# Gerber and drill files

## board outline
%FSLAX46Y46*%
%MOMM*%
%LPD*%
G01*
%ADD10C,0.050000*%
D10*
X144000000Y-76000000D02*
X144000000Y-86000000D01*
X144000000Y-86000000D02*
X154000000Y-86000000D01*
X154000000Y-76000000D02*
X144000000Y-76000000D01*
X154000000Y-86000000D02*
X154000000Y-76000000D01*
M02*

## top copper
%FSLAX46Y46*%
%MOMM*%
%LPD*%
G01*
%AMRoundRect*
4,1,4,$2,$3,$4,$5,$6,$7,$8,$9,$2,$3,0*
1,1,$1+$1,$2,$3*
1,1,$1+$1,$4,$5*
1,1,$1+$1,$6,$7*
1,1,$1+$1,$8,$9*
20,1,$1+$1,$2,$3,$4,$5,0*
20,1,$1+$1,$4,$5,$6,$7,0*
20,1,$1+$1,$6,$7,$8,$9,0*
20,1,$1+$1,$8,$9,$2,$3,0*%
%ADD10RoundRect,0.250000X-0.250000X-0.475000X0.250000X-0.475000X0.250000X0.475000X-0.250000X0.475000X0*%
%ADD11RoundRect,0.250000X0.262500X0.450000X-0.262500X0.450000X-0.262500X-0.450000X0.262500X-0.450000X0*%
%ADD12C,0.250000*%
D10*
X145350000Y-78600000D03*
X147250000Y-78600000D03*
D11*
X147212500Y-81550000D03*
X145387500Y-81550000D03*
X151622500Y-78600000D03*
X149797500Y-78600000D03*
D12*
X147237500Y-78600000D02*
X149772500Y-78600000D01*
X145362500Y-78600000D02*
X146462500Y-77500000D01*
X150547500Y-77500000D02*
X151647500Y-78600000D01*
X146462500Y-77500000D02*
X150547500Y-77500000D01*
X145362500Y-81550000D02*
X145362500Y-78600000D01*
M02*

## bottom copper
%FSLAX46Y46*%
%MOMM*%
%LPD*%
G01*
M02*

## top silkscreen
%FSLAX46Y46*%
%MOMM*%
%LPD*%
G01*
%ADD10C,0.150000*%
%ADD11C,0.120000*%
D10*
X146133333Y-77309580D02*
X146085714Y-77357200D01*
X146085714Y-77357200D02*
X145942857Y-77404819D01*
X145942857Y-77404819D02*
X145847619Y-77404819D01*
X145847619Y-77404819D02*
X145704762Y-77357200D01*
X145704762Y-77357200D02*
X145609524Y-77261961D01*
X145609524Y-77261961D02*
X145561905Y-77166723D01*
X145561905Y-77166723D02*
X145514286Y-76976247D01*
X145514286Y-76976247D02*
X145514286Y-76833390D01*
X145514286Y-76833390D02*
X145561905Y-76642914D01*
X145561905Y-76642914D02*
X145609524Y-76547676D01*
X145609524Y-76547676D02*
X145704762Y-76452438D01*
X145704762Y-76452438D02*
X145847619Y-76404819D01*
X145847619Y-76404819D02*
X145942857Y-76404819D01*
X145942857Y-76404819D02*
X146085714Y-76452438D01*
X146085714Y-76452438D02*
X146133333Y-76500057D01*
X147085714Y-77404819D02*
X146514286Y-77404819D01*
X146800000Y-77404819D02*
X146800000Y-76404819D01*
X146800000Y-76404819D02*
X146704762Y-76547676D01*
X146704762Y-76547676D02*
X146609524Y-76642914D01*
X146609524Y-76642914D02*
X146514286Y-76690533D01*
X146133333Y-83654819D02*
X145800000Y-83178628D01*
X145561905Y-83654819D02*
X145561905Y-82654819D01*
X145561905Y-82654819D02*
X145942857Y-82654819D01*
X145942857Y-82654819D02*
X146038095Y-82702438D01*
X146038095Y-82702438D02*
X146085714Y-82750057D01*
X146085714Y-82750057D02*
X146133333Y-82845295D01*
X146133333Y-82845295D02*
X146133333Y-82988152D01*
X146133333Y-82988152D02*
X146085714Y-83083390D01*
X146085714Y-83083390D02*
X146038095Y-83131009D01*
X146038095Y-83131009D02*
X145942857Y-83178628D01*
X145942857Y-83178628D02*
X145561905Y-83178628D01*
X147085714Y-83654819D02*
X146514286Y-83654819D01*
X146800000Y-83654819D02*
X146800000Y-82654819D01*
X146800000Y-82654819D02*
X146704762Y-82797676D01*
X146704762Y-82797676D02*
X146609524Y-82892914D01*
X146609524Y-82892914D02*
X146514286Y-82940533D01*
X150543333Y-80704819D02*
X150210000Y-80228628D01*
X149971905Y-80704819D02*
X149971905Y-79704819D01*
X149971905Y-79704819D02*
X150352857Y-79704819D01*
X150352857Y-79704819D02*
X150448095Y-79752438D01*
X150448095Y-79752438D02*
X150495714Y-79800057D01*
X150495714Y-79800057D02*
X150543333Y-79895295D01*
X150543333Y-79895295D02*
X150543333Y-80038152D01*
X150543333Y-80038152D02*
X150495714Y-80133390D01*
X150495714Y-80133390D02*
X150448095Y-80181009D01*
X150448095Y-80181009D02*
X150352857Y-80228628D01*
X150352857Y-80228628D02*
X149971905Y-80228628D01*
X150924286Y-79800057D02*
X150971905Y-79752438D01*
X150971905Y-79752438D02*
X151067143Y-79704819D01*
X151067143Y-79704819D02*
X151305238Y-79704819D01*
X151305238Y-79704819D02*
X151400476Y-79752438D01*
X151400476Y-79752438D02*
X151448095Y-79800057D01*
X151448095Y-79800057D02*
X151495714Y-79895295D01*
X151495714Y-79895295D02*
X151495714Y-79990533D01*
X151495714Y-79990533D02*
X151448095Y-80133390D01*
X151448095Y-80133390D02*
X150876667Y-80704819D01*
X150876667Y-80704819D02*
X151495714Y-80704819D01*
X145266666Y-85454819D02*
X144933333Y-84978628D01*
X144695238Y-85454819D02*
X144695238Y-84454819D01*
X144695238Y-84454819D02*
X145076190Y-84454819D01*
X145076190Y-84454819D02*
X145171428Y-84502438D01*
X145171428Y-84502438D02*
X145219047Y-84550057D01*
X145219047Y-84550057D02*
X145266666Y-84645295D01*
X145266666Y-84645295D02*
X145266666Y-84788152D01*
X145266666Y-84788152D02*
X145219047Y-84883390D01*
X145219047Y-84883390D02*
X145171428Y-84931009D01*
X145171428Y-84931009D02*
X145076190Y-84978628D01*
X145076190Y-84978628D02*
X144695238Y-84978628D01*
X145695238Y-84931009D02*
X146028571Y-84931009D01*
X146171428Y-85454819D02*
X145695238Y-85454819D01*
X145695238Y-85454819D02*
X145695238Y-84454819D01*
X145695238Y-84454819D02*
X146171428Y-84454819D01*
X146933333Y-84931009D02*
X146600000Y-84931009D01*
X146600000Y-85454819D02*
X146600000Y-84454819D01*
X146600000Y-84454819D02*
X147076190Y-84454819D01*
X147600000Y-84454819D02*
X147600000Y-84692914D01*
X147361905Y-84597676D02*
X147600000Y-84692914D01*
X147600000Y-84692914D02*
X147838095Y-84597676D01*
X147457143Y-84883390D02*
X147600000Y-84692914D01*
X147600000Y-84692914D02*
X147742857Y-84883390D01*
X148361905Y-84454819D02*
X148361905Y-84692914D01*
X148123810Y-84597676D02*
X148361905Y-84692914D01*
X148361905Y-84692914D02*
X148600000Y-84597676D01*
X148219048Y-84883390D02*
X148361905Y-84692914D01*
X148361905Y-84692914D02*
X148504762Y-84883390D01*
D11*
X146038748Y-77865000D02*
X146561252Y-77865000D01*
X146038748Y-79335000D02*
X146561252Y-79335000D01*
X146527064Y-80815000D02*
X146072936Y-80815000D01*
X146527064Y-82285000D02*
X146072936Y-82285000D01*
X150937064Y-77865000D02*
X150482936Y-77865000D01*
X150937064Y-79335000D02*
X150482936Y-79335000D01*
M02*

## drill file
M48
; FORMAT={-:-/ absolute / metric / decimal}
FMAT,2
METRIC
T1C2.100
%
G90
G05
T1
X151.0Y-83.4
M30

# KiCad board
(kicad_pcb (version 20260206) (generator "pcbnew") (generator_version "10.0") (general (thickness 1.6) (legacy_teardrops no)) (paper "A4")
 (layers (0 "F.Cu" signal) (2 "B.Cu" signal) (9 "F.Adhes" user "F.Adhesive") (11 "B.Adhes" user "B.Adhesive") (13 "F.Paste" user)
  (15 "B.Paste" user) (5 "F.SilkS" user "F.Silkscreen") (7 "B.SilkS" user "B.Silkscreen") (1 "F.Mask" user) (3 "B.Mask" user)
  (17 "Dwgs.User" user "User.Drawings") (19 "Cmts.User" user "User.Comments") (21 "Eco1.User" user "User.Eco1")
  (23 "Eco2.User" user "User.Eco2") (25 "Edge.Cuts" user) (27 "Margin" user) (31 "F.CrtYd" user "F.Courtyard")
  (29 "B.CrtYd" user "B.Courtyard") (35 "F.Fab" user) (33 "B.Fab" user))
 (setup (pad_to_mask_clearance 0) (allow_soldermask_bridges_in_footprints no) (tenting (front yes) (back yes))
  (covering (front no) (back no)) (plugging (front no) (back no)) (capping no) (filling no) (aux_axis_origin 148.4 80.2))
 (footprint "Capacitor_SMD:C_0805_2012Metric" (layer "F.Cu") (at 146.3 78.6)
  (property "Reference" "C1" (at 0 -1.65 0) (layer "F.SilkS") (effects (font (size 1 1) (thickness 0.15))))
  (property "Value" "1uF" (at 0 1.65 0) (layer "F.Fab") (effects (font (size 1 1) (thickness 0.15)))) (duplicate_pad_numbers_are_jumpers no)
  (fp_line (start -0.261252 -0.735) (end 0.261252 -0.735) (stroke (width 0.12) (type solid)) (layer "F.SilkS"))
  (fp_line (start -0.261252 0.735) (end 0.261252 0.735) (stroke (width 0.12) (type solid)) (layer "F.SilkS"))
  (pad "1" smd roundrect (at -0.95 0) (size 1 1.45) (layers "F.Cu" "F.Mask" "F.Paste") (roundrect_rratio 0.25) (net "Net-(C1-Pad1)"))
  (pad "2" smd roundrect (at 0.95 0) (size 1 1.45) (layers "F.Cu" "F.Mask" "F.Paste") (roundrect_rratio 0.25) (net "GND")))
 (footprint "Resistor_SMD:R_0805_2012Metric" (layer "F.Cu") (at 146.3 81.55 180)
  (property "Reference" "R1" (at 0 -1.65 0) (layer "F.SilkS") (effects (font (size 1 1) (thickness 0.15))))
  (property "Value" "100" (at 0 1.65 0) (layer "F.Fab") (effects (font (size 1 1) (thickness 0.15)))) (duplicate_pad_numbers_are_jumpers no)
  (fp_line (start -0.227064 0.735) (end 0.227064 0.735) (stroke (width 0.12) (type solid)) (layer "F.SilkS"))
  (fp_line (start -0.227064 -0.735) (end 0.227064 -0.735) (stroke (width 0.12) (type solid)) (layer "F.SilkS"))
  (pad "1" smd roundrect (at -0.9125 0 180) (size 1.025 1.4) (layers "F.Cu" "F.Mask" "F.Paste") (roundrect_rratio 0.243902) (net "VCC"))
  (pad "2" smd roundrect (at 0.9125 0 180) (size 1.025 1.4) (layers "F.Cu" "F.Mask" "F.Paste") (roundrect_rratio 0.243902)
   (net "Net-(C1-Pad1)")))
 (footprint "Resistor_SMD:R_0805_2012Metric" (layer "F.Cu") (at 150.71 78.6 180)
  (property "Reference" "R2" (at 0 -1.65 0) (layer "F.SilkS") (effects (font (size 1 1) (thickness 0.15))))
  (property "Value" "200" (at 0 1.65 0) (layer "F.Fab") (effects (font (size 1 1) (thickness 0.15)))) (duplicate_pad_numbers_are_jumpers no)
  (fp_line (start -0.227064 0.735) (end 0.227064 0.735) (stroke (width 0.12) (type solid)) (layer "F.SilkS"))
  (fp_line (start -0.227064 -0.735) (end 0.227064 -0.735) (stroke (width 0.12) (type solid)) (layer "F.SilkS"))
  (pad "1" smd roundrect (at -0.9125 0 180) (size 1.025 1.4) (layers "F.Cu" "F.Mask" "F.Paste") (roundrect_rratio 0.243902)
   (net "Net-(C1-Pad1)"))
  (pad "2" smd roundrect (at 0.9125 0 180) (size 1.025 1.4) (layers "F.Cu" "F.Mask" "F.Paste") (roundrect_rratio 0.243902) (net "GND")))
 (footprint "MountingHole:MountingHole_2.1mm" (layer "F.Cu") (at 151 83.4)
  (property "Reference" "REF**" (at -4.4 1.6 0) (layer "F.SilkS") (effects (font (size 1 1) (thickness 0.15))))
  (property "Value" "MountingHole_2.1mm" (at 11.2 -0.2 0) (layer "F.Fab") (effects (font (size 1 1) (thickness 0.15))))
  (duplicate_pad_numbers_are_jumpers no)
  (pad "" np_thru_hole circle (at 0 0) (size 2.1 2.1) (drill 2.1) (layers "*.Cu" "*.Mask")))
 (gr_line (start 144 76) (end 144 86) (stroke (width 0.05) (type solid)) (layer "Edge.Cuts"))
 (gr_line (start 144 86) (end 154 86) (stroke (width 0.05) (type solid)) (layer "Edge.Cuts"))
 (gr_line (start 154 76) (end 144 76) (stroke (width 0.05) (type solid)) (layer "Edge.Cuts"))
 (gr_line (start 154 86) (end 154 76) (stroke (width 0.05) (type solid)) (layer "Edge.Cuts"))
 (segment (start 147.2375 78.6) (end 149.7725 78.6) (width 0.25) (layer "F.Cu") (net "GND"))
 (segment (start 145.3625 78.6) (end 146.4625 77.5) (width 0.25) (layer "F.Cu") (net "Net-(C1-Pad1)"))
 (segment (start 150.5475 77.5) (end 151.6475 78.6) (width 0.25) (layer "F.Cu") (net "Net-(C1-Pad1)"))
 (segment (start 146.4625 77.5) (end 150.5475 77.5) (width 0.25) (layer "F.Cu") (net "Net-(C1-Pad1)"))
 (segment (start 145.3625 81.55) (end 145.3625 78.6) (width 0.25) (layer "F.Cu") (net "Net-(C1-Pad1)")))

